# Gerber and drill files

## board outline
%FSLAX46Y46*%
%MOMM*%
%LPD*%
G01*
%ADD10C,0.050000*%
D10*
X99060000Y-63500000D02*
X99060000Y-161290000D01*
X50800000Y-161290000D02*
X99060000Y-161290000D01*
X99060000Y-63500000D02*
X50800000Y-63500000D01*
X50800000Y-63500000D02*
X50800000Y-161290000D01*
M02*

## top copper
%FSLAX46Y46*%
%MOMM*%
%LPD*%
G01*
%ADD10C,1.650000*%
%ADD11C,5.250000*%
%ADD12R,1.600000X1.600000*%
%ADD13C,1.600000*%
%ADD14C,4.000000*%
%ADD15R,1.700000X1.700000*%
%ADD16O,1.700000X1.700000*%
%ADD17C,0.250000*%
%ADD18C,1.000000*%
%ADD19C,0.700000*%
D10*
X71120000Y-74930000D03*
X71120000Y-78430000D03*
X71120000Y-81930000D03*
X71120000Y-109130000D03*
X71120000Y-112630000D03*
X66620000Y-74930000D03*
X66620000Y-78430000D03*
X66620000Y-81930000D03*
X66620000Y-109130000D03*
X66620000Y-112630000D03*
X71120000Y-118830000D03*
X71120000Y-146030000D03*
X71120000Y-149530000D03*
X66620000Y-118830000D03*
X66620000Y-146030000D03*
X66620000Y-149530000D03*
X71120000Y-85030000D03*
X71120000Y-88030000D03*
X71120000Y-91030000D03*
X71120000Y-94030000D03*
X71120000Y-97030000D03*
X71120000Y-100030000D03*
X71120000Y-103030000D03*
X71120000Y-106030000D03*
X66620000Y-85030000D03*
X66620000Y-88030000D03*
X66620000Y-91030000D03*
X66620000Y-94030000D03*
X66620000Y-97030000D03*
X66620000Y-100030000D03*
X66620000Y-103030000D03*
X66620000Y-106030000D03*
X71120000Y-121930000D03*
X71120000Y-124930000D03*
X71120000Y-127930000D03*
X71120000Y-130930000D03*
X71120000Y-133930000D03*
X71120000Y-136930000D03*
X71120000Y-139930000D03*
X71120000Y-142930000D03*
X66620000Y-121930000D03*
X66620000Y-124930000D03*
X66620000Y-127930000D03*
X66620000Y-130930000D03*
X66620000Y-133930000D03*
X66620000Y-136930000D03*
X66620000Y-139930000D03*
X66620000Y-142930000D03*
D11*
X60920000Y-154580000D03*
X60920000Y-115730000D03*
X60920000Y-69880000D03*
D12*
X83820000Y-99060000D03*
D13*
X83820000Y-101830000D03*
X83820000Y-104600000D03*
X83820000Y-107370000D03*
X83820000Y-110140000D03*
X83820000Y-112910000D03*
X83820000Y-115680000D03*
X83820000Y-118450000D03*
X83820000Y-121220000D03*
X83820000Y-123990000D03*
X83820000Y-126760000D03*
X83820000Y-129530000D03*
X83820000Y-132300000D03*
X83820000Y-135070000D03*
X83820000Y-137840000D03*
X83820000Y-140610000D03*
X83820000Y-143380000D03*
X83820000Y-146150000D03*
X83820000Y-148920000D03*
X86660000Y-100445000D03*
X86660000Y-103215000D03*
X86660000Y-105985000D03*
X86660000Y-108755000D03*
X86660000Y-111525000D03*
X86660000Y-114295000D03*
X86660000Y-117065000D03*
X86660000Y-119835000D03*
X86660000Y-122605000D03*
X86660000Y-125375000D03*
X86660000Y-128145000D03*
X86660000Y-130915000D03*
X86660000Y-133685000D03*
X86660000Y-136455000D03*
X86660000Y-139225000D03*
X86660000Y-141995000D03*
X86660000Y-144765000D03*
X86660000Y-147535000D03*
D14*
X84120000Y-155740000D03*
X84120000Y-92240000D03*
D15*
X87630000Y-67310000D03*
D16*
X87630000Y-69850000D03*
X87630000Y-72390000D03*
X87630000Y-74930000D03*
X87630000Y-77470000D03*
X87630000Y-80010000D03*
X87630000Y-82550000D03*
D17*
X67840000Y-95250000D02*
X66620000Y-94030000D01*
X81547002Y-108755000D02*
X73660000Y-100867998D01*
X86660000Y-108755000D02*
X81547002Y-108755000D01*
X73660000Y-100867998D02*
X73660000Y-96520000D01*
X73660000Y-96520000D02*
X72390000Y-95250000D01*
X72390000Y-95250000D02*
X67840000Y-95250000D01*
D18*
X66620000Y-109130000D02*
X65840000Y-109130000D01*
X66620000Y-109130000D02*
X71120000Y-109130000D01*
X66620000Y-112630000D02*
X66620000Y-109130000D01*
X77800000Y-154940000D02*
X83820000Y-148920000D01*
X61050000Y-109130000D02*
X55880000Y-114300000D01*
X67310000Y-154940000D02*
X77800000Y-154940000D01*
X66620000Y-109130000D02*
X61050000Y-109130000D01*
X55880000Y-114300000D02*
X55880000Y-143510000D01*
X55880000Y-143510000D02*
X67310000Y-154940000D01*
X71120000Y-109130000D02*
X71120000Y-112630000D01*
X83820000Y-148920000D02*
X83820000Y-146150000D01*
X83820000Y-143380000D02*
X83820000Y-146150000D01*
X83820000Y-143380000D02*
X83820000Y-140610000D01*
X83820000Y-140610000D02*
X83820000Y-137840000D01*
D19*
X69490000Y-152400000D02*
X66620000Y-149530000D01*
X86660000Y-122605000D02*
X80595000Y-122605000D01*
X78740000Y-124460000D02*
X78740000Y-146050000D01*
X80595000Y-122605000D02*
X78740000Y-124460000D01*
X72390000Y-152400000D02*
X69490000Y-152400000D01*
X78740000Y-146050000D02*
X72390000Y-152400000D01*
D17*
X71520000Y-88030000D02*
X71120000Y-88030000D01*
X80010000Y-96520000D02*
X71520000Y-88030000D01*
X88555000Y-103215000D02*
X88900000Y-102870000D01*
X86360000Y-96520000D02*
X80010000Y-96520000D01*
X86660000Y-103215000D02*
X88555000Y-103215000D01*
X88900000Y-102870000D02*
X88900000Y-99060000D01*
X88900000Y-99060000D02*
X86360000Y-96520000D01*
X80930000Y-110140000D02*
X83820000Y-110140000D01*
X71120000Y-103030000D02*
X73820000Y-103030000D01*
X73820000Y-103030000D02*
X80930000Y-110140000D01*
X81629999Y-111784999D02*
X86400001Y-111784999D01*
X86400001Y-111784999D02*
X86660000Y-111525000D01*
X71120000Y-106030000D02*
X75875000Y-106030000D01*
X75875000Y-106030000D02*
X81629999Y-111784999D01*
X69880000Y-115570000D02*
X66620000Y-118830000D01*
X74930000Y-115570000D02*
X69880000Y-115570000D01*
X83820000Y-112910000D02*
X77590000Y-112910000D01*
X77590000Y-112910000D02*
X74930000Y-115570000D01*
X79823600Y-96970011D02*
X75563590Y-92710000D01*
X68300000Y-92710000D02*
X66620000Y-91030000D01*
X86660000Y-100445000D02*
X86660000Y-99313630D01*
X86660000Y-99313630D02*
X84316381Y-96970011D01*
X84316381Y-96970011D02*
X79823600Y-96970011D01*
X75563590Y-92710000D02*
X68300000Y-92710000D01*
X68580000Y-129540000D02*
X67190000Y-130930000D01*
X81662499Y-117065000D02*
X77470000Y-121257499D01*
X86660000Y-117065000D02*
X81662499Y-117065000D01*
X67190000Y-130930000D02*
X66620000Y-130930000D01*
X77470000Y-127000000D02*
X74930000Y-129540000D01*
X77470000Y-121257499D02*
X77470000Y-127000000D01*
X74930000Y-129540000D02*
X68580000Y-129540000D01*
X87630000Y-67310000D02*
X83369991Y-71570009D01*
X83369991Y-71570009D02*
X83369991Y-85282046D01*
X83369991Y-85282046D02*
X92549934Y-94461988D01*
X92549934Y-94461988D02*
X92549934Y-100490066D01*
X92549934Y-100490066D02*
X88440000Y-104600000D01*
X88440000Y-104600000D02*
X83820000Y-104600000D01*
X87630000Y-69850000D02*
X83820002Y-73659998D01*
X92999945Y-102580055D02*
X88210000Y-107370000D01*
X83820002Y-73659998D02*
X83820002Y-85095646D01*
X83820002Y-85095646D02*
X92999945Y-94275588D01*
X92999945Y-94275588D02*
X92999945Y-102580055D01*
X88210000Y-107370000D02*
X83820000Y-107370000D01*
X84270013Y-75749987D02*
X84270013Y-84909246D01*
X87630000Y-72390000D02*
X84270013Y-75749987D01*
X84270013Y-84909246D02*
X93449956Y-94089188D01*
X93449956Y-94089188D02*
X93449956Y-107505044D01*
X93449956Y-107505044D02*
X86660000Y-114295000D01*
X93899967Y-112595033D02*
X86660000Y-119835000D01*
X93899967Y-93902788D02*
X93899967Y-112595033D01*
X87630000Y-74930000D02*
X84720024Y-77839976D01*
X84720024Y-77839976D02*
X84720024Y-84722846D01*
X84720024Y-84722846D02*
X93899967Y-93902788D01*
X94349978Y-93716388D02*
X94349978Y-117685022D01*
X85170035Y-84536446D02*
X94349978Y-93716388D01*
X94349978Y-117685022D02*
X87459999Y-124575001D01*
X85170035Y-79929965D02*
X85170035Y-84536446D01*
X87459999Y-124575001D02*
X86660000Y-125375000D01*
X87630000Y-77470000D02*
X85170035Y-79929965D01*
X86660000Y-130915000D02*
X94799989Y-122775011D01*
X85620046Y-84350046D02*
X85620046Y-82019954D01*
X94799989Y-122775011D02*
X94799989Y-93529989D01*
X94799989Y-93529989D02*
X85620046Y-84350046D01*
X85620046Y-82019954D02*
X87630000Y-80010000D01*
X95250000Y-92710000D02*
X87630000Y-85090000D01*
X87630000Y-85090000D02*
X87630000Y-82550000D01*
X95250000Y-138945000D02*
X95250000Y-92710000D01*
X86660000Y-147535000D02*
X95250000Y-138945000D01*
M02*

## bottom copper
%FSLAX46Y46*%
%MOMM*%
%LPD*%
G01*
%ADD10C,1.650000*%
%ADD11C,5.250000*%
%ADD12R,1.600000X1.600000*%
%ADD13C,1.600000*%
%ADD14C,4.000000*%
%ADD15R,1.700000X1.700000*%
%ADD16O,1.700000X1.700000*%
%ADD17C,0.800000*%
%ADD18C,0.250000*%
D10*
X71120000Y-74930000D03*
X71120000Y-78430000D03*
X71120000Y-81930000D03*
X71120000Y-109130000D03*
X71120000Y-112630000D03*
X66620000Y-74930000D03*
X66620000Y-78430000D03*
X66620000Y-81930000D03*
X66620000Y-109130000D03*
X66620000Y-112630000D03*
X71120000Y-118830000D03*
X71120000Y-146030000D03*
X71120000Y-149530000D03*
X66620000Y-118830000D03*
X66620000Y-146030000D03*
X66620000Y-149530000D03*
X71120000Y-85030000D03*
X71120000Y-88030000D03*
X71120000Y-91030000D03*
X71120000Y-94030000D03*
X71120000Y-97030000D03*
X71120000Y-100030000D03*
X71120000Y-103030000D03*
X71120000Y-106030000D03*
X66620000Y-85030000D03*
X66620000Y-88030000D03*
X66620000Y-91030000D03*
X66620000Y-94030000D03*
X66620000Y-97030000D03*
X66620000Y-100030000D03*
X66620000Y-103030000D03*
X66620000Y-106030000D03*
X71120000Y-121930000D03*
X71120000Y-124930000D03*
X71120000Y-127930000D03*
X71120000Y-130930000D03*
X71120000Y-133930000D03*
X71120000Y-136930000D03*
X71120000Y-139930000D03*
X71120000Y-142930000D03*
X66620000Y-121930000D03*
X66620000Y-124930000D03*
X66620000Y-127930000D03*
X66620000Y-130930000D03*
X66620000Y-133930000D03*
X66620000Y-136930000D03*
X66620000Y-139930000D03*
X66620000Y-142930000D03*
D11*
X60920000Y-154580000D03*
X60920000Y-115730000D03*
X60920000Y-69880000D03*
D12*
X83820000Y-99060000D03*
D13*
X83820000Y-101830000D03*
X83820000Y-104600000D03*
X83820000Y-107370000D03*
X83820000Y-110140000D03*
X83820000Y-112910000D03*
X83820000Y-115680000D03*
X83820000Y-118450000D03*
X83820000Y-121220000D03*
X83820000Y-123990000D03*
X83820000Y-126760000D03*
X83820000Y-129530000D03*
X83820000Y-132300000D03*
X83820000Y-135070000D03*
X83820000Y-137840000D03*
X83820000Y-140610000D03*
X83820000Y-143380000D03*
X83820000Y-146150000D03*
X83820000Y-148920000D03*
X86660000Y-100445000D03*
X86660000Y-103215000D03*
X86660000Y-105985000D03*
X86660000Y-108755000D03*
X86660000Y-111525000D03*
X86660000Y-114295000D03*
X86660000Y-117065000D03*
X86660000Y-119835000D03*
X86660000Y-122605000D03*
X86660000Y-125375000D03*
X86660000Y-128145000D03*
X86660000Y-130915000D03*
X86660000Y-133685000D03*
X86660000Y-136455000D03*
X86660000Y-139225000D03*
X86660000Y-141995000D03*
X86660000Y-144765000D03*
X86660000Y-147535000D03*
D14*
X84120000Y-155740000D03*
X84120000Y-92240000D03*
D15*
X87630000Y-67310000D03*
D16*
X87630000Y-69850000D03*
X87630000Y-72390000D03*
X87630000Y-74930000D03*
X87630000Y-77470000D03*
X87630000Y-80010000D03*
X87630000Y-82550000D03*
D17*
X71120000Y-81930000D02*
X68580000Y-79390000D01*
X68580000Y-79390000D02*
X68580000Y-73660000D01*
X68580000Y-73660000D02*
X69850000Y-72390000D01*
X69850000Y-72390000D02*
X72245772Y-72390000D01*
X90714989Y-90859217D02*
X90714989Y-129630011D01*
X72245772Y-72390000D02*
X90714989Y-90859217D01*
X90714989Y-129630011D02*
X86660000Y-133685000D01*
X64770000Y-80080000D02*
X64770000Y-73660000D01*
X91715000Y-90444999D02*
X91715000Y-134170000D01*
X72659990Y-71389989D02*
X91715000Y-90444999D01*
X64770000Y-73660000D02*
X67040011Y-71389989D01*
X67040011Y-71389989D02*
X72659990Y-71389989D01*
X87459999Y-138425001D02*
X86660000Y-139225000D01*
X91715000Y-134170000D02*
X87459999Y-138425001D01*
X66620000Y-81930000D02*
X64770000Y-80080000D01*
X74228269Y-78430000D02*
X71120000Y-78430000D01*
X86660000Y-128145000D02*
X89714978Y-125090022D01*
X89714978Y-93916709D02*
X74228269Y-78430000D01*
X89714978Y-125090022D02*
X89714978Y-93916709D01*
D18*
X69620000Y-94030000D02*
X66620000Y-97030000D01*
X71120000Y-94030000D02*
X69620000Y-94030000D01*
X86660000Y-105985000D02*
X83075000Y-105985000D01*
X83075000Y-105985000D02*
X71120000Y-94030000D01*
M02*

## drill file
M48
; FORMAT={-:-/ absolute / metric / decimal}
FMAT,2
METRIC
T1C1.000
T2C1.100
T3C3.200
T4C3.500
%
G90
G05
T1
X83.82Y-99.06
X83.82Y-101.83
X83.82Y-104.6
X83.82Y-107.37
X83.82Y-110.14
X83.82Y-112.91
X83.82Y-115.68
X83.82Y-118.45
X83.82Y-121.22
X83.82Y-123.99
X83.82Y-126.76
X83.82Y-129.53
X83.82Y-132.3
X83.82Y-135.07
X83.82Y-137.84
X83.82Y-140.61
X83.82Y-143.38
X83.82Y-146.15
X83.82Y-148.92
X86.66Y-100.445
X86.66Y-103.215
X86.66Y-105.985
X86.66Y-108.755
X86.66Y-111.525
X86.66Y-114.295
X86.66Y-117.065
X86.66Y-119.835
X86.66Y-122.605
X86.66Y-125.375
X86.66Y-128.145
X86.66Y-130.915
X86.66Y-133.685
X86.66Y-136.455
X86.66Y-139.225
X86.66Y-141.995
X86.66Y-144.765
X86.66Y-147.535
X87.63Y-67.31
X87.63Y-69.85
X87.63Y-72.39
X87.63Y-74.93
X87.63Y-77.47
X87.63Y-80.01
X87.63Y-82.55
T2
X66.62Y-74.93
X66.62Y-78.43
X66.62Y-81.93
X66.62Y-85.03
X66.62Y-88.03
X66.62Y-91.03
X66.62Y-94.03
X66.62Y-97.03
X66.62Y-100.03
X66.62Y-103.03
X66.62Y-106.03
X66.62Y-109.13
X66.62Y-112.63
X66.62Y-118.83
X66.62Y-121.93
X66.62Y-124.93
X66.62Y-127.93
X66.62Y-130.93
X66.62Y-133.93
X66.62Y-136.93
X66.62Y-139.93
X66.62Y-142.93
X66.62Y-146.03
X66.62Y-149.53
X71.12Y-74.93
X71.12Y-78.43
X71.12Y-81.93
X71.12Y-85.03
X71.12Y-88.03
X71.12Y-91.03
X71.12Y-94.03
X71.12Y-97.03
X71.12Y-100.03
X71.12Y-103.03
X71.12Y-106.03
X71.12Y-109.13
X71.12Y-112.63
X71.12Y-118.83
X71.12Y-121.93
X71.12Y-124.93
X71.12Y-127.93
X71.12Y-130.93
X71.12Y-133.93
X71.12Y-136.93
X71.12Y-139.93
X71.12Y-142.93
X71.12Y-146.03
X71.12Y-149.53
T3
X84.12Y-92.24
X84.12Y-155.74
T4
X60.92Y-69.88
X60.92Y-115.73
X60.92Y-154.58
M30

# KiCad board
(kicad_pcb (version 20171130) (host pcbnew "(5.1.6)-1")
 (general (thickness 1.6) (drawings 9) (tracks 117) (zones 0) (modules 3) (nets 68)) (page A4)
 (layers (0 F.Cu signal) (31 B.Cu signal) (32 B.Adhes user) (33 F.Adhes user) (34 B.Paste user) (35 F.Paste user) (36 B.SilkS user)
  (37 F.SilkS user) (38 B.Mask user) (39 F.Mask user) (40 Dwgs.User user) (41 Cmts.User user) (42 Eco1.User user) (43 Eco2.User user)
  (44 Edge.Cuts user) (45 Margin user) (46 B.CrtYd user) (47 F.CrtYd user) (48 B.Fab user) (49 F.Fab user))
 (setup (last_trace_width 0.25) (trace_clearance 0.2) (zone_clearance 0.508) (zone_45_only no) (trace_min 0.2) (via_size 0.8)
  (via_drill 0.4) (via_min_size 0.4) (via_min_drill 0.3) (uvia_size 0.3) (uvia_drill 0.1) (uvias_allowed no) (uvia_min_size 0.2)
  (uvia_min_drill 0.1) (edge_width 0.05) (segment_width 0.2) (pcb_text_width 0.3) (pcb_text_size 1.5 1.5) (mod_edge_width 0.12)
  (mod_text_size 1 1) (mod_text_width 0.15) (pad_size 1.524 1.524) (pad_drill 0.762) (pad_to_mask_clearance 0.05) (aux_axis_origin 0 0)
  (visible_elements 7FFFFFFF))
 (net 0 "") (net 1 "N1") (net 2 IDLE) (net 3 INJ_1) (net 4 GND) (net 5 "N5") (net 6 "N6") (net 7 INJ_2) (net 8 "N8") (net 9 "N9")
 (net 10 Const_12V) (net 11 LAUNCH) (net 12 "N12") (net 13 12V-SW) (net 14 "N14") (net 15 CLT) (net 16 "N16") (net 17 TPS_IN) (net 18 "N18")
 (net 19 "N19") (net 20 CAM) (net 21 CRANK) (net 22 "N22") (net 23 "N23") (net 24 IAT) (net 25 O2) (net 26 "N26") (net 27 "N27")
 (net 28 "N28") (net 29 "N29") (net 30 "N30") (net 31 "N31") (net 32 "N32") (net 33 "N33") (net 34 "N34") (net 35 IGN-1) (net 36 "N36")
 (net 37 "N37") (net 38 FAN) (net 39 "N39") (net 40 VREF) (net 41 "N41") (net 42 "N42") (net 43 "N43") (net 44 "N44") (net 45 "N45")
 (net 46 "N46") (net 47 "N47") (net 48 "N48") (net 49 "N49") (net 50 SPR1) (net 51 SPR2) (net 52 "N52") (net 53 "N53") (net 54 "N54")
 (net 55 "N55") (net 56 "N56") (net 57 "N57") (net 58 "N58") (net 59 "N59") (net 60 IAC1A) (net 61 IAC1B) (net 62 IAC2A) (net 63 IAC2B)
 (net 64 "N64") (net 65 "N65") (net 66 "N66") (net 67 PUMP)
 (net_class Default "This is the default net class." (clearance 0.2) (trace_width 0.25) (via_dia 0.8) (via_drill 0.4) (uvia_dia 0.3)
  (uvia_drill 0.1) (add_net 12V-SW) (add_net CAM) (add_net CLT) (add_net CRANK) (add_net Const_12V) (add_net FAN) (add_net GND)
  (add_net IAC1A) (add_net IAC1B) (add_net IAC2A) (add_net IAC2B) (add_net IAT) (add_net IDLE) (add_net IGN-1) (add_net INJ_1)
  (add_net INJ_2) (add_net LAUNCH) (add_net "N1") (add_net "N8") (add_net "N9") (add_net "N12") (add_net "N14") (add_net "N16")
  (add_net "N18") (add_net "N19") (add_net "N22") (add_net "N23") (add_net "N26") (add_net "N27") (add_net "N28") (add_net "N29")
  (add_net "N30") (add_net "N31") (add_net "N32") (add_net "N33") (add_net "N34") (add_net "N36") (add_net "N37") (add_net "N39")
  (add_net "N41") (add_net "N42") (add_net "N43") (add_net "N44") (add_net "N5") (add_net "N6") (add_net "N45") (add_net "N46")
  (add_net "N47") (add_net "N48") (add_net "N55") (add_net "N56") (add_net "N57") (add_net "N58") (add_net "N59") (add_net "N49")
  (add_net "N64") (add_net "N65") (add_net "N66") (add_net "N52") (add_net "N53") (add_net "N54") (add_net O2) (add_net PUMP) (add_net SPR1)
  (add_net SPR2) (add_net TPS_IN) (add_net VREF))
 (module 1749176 (layer F.Cu) (at 71.12 74.93 180)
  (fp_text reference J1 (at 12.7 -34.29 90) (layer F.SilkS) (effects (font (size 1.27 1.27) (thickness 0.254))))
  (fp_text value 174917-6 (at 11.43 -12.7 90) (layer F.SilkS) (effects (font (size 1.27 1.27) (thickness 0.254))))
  (pad 1 thru_hole circle (at 0 0 270) (size 1.65 1.65) (drill 1.1) (layers *.Cu *.Mask F.SilkS) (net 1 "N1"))
  (pad 2 thru_hole circle (at 0 -3.5 270) (size 1.65 1.65) (drill 1.1) (layers *.Cu *.Mask F.SilkS) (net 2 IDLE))
  (pad 3 thru_hole circle (at 0 -7 270) (size 1.65 1.65) (drill 1.1) (layers *.Cu *.Mask F.SilkS) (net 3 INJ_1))
  (pad 4 thru_hole circle (at 0 -34.2 270) (size 1.65 1.65) (drill 1.1) (layers *.Cu *.Mask F.SilkS) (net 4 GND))
  (pad 5 thru_hole circle (at 0 -37.7 270) (size 1.65 1.65) (drill 1.1) (layers *.Cu *.Mask F.SilkS) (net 4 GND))
  (pad 6 thru_hole circle (at 4.5 0 270) (size 1.65 1.65) (drill 1.1) (layers *.Cu *.Mask F.SilkS) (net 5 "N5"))
  (pad 7 thru_hole circle (at 4.5 -3.5 270) (size 1.65 1.65) (drill 1.1) (layers *.Cu *.Mask F.SilkS) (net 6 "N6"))
  (pad 8 thru_hole circle (at 4.5 -7 270) (size 1.65 1.65) (drill 1.1) (layers *.Cu *.Mask F.SilkS) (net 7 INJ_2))
  (pad 9 thru_hole circle (at 4.5 -34.2 270) (size 1.65 1.65) (drill 1.1) (layers *.Cu *.Mask F.SilkS) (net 4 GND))
  (pad 10 thru_hole circle (at 4.5 -37.7 270) (size 1.65 1.65) (drill 1.1) (layers *.Cu *.Mask F.SilkS) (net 4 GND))
  (pad 11 thru_hole circle (at 0 -43.9 270) (size 1.65 1.65) (drill 1.1) (layers *.Cu *.Mask F.SilkS) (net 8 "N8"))
  (pad 12 thru_hole circle (at 0 -71.1 270) (size 1.65 1.65) (drill 1.1) (layers *.Cu *.Mask F.SilkS) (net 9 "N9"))
  (pad 13 thru_hole circle (at 0 -74.6 270) (size 1.65 1.65) (drill 1.1) (layers *.Cu *.Mask F.SilkS) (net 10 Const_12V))
  (pad 14 thru_hole circle (at 4.5 -43.9 270) (size 1.65 1.65) (drill 1.1) (layers *.Cu *.Mask F.SilkS) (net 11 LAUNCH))
  (pad 15 thru_hole circle (at 4.5 -71.1 270) (size 1.65 1.65) (drill 1.1) (layers *.Cu *.Mask F.SilkS) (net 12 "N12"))
  (pad 16 thru_hole circle (at 4.5 -74.6 270) (size 1.65 1.65) (drill 1.1) (layers *.Cu *.Mask F.SilkS) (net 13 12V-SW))
  (pad 17 thru_hole circle (at 0 -10.1 270) (size 1.65 1.65) (drill 1.1) (layers *.Cu *.Mask F.SilkS) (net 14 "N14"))
  (pad 18 thru_hole circle (at 0 -13.1 270) (size 1.65 1.65) (drill 1.1) (layers *.Cu *.Mask F.SilkS) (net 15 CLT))
  (pad 19 thru_hole circle (at 0 -16.1 270) (size 1.65 1.65) (drill 1.1) (layers *.Cu *.Mask F.SilkS) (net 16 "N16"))
  (pad 20 thru_hole circle (at 0 -19.1 270) (size 1.65 1.65) (drill 1.1) (layers *.Cu *.Mask F.SilkS) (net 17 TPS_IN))
  (pad 21 thru_hole circle (at 0 -22.1 270) (size 1.65 1.65) (drill 1.1) (layers *.Cu *.Mask F.SilkS) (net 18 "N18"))
  (pad 22 thru_hole circle (at 0 -25.1 270) (size 1.65 1.65) (drill 1.1) (layers *.Cu *.Mask F.SilkS) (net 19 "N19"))
  (pad 23 thru_hole circle (at 0 -28.1 270) (size 1.65 1.65) (drill 1.1) (layers *.Cu *.Mask F.SilkS) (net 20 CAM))
  (pad 24 thru_hole circle (at 0 -31.1 270) (size 1.65 1.65) (drill 1.1) (layers *.Cu *.Mask F.SilkS) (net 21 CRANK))
  (pad 25 thru_hole circle (at 4.5 -10.1 270) (size 1.65 1.65) (drill 1.1) (layers *.Cu *.Mask F.SilkS) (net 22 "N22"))
  (pad 26 thru_hole circle (at 4.5 -13.1 270) (size 1.65 1.65) (drill 1.1) (layers *.Cu *.Mask F.SilkS) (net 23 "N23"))
  (pad 27 thru_hole circle (at 4.5 -16.1 270) (size 1.65 1.65) (drill 1.1) (layers *.Cu *.Mask F.SilkS) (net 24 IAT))
  (pad 28 thru_hole circle (at 4.5 -19.1 270) (size 1.65 1.65) (drill 1.1) (layers *.Cu *.Mask F.SilkS) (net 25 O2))
  (pad 29 thru_hole circle (at 4.5 -22.1 270) (size 1.65 1.65) (drill 1.1) (layers *.Cu *.Mask F.SilkS) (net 17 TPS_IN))
  (pad 30 thru_hole circle (at 4.5 -25.1 270) (size 1.65 1.65) (drill 1.1) (layers *.Cu *.Mask F.SilkS) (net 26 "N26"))
  (pad 31 thru_hole circle (at 4.5 -28.1 270) (size 1.65 1.65) (drill 1.1) (layers *.Cu *.Mask F.SilkS) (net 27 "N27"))
  (pad 32 thru_hole circle (at 4.5 -31.1 270) (size 1.65 1.65) (drill 1.1) (layers *.Cu *.Mask F.SilkS) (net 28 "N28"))
  (pad 33 thru_hole circle (at 0 -47 270) (size 1.65 1.65) (drill 1.1) (layers *.Cu *.Mask F.SilkS) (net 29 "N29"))
  (pad 34 thru_hole circle (at 0 -50 270) (size 1.65 1.65) (drill 1.1) (layers *.Cu *.Mask F.SilkS) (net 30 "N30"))
  (pad 35 thru_hole circle (at 0 -53 270) (size 1.65 1.65) (drill 1.1) (layers *.Cu *.Mask F.SilkS) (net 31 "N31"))
  (pad 36 thru_hole circle (at 0 -56 270) (size 1.65 1.65) (drill 1.1) (layers *.Cu *.Mask F.SilkS) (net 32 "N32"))
  (pad 37 thru_hole circle (at 0 -59 270) (size 1.65 1.65) (drill 1.1) (layers *.Cu *.Mask F.SilkS) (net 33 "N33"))
  (pad 38 thru_hole circle (at 0 -62 270) (size 1.65 1.65) (drill 1.1) (layers *.Cu *.Mask F.SilkS) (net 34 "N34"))
  (pad 39 thru_hole circle (at 0 -65 270) (size 1.65 1.65) (drill 1.1) (layers *.Cu *.Mask F.SilkS) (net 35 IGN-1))
  (pad 40 thru_hole circle (at 0 -68 270) (size 1.65 1.65) (drill 1.1) (layers *.Cu *.Mask F.SilkS) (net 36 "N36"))
  (pad 41 thru_hole circle (at 4.5 -47 270) (size 1.65 1.65) (drill 1.1) (layers *.Cu *.Mask F.SilkS) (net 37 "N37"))
  (pad 42 thru_hole circle (at 4.5 -50 270) (size 1.65 1.65) (drill 1.1) (layers *.Cu *.Mask F.SilkS) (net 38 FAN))
  (pad 43 thru_hole circle (at 4.5 -53 270) (size 1.65 1.65) (drill 1.1) (layers *.Cu *.Mask F.SilkS) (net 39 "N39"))
  (pad 44 thru_hole circle (at 4.5 -56 270) (size 1.65 1.65) (drill 1.1) (layers *.Cu *.Mask F.SilkS) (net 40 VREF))
  (pad 45 thru_hole circle (at 4.5 -59 270) (size 1.65 1.65) (drill 1.1) (layers *.Cu *.Mask F.SilkS) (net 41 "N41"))
  (pad 46 thru_hole circle (at 4.5 -62 270) (size 1.65 1.65) (drill 1.1) (layers *.Cu *.Mask F.SilkS) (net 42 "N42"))
  (pad 47 thru_hole circle (at 4.5 -65 270) (size 1.65 1.65) (drill 1.1) (layers *.Cu *.Mask F.SilkS) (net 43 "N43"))
  (pad 48 thru_hole circle (at 4.5 -68 270) (size 1.65 1.65) (drill 1.1) (layers *.Cu *.Mask F.SilkS) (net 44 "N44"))
  (pad MH1 thru_hole circle (at 10.2 -79.65 270) (size 5.25 5.25) (drill 3.5) (layers *.Cu *.Mask F.SilkS) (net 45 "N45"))
  (pad MH2 thru_hole circle (at 10.2 -40.8 270) (size 5.25 5.25) (drill 3.5) (layers *.Cu *.Mask F.SilkS) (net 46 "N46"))
  (pad MH3 thru_hole circle (at 10.2 5.05 270) (size 5.25 5.25) (drill 3.5) (layers *.Cu *.Mask F.SilkS) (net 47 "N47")))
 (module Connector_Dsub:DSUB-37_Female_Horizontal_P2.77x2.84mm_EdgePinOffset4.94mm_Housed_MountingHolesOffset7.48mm (layer F.Cu)
  (at 83.82 99.06 90)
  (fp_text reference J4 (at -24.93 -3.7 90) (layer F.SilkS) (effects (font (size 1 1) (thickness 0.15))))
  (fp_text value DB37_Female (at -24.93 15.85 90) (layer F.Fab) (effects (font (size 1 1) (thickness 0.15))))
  (pad 1 thru_hole rect (at 0 0 90) (size 1.6 1.6) (drill 1) (layers *.Cu *.Mask) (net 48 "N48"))
  (pad 2 thru_hole circle (at -2.77 0 90) (size 1.6 1.6) (drill 1) (layers *.Cu *.Mask) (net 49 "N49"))
  (pad 3 thru_hole circle (at -5.54 0 90) (size 1.6 1.6) (drill 1) (layers *.Cu *.Mask) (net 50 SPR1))
  (pad 4 thru_hole circle (at -8.31 0 90) (size 1.6 1.6) (drill 1) (layers *.Cu *.Mask) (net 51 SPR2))
  (pad 5 thru_hole circle (at -11.08 0 90) (size 1.6 1.6) (drill 1) (layers *.Cu *.Mask) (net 20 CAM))
  (pad 6 thru_hole circle (at -13.85 0 90) (size 1.6 1.6) (drill 1) (layers *.Cu *.Mask) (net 11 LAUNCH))
  (pad 7 thru_hole circle (at -16.62 0 90) (size 1.6 1.6) (drill 1) (layers *.Cu *.Mask) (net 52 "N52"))
  (pad 8 thru_hole circle (at -19.39 0 90) (size 1.6 1.6) (drill 1) (layers *.Cu *.Mask) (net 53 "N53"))
  (pad 9 thru_hole circle (at -22.16 0 90) (size 1.6 1.6) (drill 1) (layers *.Cu *.Mask) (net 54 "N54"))
  (pad 10 thru_hole circle (at -24.93 0 90) (size 1.6 1.6) (drill 1) (layers *.Cu *.Mask) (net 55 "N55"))
  (pad 11 thru_hole circle (at -27.7 0 90) (size 1.6 1.6) (drill 1) (layers *.Cu *.Mask) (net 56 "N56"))
  (pad 12 thru_hole circle (at -30.47 0 90) (size 1.6 1.6) (drill 1) (layers *.Cu *.Mask) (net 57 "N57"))
  (pad 13 thru_hole circle (at -33.24 0 90) (size 1.6 1.6) (drill 1) (layers *.Cu *.Mask) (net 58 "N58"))
  (pad 14 thru_hole circle (at -36.01 0 90) (size 1.6 1.6) (drill 1) (layers *.Cu *.Mask) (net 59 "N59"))
  (pad 15 thru_hole circle (at -38.78 0 90) (size 1.6 1.6) (drill 1) (layers *.Cu *.Mask) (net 4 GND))
  (pad 16 thru_hole circle (at -41.55 0 90) (size 1.6 1.6) (drill 1) (layers *.Cu *.Mask) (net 4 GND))
  (pad 17 thru_hole circle (at -44.32 0 90) (size 1.6 1.6) (drill 1) (layers *.Cu *.Mask) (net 4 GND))
  (pad 18 thru_hole circle (at -47.09 0 90) (size 1.6 1.6) (drill 1) (layers *.Cu *.Mask) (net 4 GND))
  (pad 19 thru_hole circle (at -49.86 0 90) (size 1.6 1.6) (drill 1) (layers *.Cu *.Mask) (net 4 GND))
  (pad 20 thru_hole circle (at -1.385 2.84 90) (size 1.6 1.6) (drill 1) (layers *.Cu *.Mask) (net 24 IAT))
  (pad 21 thru_hole circle (at -4.155 2.84 90) (size 1.6 1.6) (drill 1) (layers *.Cu *.Mask) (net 15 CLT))
  (pad 22 thru_hole circle (at -6.925 2.84 90) (size 1.6 1.6) (drill 1) (layers *.Cu *.Mask) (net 17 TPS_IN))
  (pad 23 thru_hole circle (at -9.695 2.84 90) (size 1.6 1.6) (drill 1) (layers *.Cu *.Mask) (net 25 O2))
  (pad 24 thru_hole circle (at -12.465 2.84 90) (size 1.6 1.6) (drill 1) (layers *.Cu *.Mask) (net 21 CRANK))
  (pad 25 thru_hole circle (at -15.235 2.84 90) (size 1.6 1.6) (drill 1) (layers *.Cu *.Mask) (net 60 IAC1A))
  (pad 26 thru_hole circle (at -18.005 2.84 90) (size 1.6 1.6) (drill 1) (layers *.Cu *.Mask) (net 40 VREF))
  (pad 27 thru_hole circle (at -20.775 2.84 90) (size 1.6 1.6) (drill 1) (layers *.Cu *.Mask) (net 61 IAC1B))
  (pad 28 thru_hole circle (at -23.545 2.84 90) (size 1.6 1.6) (drill 1) (layers *.Cu *.Mask) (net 13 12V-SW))
  (pad 29 thru_hole circle (at -26.315 2.84 90) (size 1.6 1.6) (drill 1) (layers *.Cu *.Mask) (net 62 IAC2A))
  (pad 30 thru_hole circle (at -29.085 2.84 90) (size 1.6 1.6) (drill 1) (layers *.Cu *.Mask) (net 2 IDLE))
  (pad 31 thru_hole circle (at -31.855 2.84 90) (size 1.6 1.6) (drill 1) (layers *.Cu *.Mask) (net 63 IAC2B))
  (pad 32 thru_hole circle (at -34.625 2.84 90) (size 1.6 1.6) (drill 1) (layers *.Cu *.Mask) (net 3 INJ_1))
  (pad 33 thru_hole circle (at -37.395 2.84 90) (size 1.6 1.6) (drill 1) (layers *.Cu *.Mask) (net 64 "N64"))
  (pad 34 thru_hole circle (at -40.165 2.84 90) (size 1.6 1.6) (drill 1) (layers *.Cu *.Mask) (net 7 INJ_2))
  (pad 35 thru_hole circle (at -42.935 2.84 90) (size 1.6 1.6) (drill 1) (layers *.Cu *.Mask) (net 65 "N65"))
  (pad 36 thru_hole circle (at -45.705 2.84 90) (size 1.6 1.6) (drill 1) (layers *.Cu *.Mask) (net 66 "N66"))
  (pad 37 thru_hole circle (at -48.475 2.84 90) (size 1.6 1.6) (drill 1) (layers *.Cu *.Mask) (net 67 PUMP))
  (pad 0 thru_hole circle (at -56.68 0.3 90) (size 4 4) (drill 3.2) (layers *.Cu *.Mask))
  (pad 0 thru_hole circle (at 6.82 0.3 90) (size 4 4) (drill 3.2) (layers *.Cu *.Mask)))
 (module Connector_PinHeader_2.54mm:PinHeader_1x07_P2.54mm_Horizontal (layer F.Cu) (at 87.63 67.31)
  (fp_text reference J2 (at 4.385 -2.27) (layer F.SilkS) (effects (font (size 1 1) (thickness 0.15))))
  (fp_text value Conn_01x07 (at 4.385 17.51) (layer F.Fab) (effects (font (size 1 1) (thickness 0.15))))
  (pad 1 thru_hole rect (at 0 0) (size 1.7 1.7) (drill 1) (layers *.Cu *.Mask) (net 50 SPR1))
  (pad 2 thru_hole oval (at 0 2.54) (size 1.7 1.7) (drill 1) (layers *.Cu *.Mask) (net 51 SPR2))
  (pad 3 thru_hole oval (at 0 5.08) (size 1.7 1.7) (drill 1) (layers *.Cu *.Mask) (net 60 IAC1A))
  (pad 4 thru_hole oval (at 0 7.62) (size 1.7 1.7) (drill 1) (layers *.Cu *.Mask) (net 61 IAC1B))
  (pad 5 thru_hole oval (at 0 10.16) (size 1.7 1.7) (drill 1) (layers *.Cu *.Mask) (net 62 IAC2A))
  (pad 6 thru_hole oval (at 0 12.7) (size 1.7 1.7) (drill 1) (layers *.Cu *.Mask) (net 63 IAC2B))
  (pad 7 thru_hole oval (at 0 15.24) (size 1.7 1.7) (drill 1) (layers *.Cu *.Mask) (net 67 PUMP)))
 (gr_line (start 99.06 63.5) (end 99.06 161.29) (layer Edge.Cuts) (width 0.05))
 (gr_line (start 50.8 161.29) (end 99.06 161.29) (layer Edge.Cuts) (width 0.05))
 (gr_line (start 99.06 63.5) (end 50.8 63.5) (layer Edge.Cuts) (width 0.05))
 (gr_line (start 50.8 63.5) (end 50.8 161.29) (layer Edge.Cuts) (width 0.05))
 (segment (start 71.12 81.93) (end 68.58 79.39) (width 0.8) (layer B.Cu) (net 3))
 (segment (start 68.58 79.39) (end 68.58 73.66) (width 0.8) (layer B.Cu) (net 3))
 (segment (start 68.58 73.66) (end 69.85 72.39) (width 0.8) (layer B.Cu) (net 3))
 (segment (start 69.85 72.39) (end 72.245772 72.39) (width 0.8) (layer B.Cu) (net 3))
 (segment (start 90.714989 90.859217) (end 90.714989 129.630011) (width 0.8) (layer B.Cu) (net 3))
 (segment (start 72.245772 72.39) (end 90.714989 90.859217) (width 0.8) (layer B.Cu) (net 3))
 (segment (start 90.714989 129.630011) (end 86.66 133.685) (width 0.8) (layer B.Cu) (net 3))
 (segment (start 64.77 80.08) (end 64.77 73.66) (width 0.8) (layer B.Cu) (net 7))
 (segment (start 91.715 90.444999) (end 91.715 134.17) (width 0.8) (layer B.Cu) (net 7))
 (segment (start 72.65999 71.389989) (end 91.715 90.444999) (width 0.8) (layer B.Cu) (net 7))
 (segment (start 64.77 73.66) (end 67.040011 71.389989) (width 0.8) (layer B.Cu) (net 7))
 (segment (start 67.040011 71.389989) (end 72.65999 71.389989) (width 0.8) (layer B.Cu) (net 7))
 (segment (start 87.459999 138.425001) (end 86.66 139.225) (width 0.8) (layer B.Cu) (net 7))
 (segment (start 91.715 134.17) (end 87.459999 138.425001) (width 0.8) (layer B.Cu) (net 7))
 (segment (start 66.62 81.93) (end 64.77 80.08) (width 0.8) (layer B.Cu) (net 7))
 (segment (start 67.84 95.25) (end 66.62 94.03) (width 0.25) (layer F.Cu) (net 25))
 (segment (start 81.547002 108.755) (end 73.66 100.867998) (width 0.25) (layer F.Cu) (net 25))
 (segment (start 86.66 108.755) (end 81.547002 108.755) (width 0.25) (layer F.Cu) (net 25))
 (segment (start 73.66 100.867998) (end 73.66 96.52) (width 0.25) (layer F.Cu) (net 25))
 (segment (start 73.66 96.52) (end 72.39 95.25) (width 0.25) (layer F.Cu) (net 25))
 (segment (start 72.39 95.25) (end 67.84 95.25) (width 0.25) (layer F.Cu) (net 25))
 (segment (start 66.62 109.13) (end 65.84 109.13) (width 1) (layer F.Cu) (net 4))
 (segment (start 66.62 109.13) (end 71.12 109.13) (width 1) (layer F.Cu) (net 4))
 (segment (start 66.62 112.63) (end 66.62 109.13) (width 1) (layer F.Cu) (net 4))
 (segment (start 77.8 154.94) (end 83.82 148.92) (width 1) (layer F.Cu) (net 4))
 (segment (start 61.05 109.13) (end 55.88 114.3) (width 1) (layer F.Cu) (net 4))
 (segment (start 67.31 154.94) (end 77.8 154.94) (width 1) (layer F.Cu) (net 4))
 (segment (start 66.62 109.13) (end 61.05 109.13) (width 1) (layer F.Cu) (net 4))
 (segment (start 55.88 114.3) (end 55.88 143.51) (width 1) (layer F.Cu) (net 4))
 (segment (start 55.88 143.51) (end 67.31 154.94) (width 1) (layer F.Cu) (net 4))
 (segment (start 71.12 109.13) (end 71.12 112.63) (width 1) (layer F.Cu) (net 4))
 (segment (start 83.82 148.92) (end 83.82 146.15) (width 1) (layer F.Cu) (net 4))
 (segment (start 83.82 143.38) (end 83.82 146.15) (width 1) (layer F.Cu) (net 4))
 (segment (start 83.82 143.38) (end 83.82 140.61) (width 1) (layer F.Cu) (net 4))
 (segment (start 83.82 140.61) (end 83.82 137.84) (width 1) (layer F.Cu) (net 4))
 (segment (start 69.49 152.4) (end 66.62 149.53) (width 0.7) (layer F.Cu) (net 13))
 (segment (start 86.66 122.605) (end 80.595 122.605) (width 0.7) (layer F.Cu) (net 13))
 (segment (start 78.74 124.46) (end 78.74 146.05) (width 0.7) (layer F.Cu) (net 13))
 (segment (start 80.595 122.605) (end 78.74 124.46) (width 0.7) (layer F.Cu) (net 13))
 (segment (start 72.39 152.4) (end 69.49 152.4) (width 0.7) (layer F.Cu) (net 13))
 (segment (start 78.74 146.05) (end 72.39 152.4) (width 0.7) (layer F.Cu) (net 13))
 (segment (start 71.52 88.03) (end 71.12 88.03) (width 0.25) (layer F.Cu) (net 15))
 (segment (start 80.01 96.52) (end 71.52 88.03) (width 0.25) (layer F.Cu) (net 15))
 (segment (start 88.555 103.215) (end 88.9 102.87) (width 0.25) (layer F.Cu) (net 15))
 (segment (start 86.36 96.52) (end 80.01 96.52) (width 0.25) (layer F.Cu) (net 15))
 (segment (start 86.66 103.215) (end 88.555 103.215) (width 0.25) (layer F.Cu) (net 15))
 (segment (start 88.9 102.87) (end 88.9 99.06) (width 0.25) (layer F.Cu) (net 15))
 (segment (start 88.9 99.06) (end 86.36 96.52) (width 0.25) (layer F.Cu) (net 15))
 (segment (start 80.93 110.14) (end 83.82 110.14) (width 0.25) (layer F.Cu) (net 20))
 (segment (start 71.12 103.03) (end 73.82 103.03) (width 0.25) (layer F.Cu) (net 20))
 (segment (start 73.82 103.03) (end 80.93 110.14) (width 0.25) (layer F.Cu) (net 20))
 (segment (start 81.629999 111.784999) (end 86.400001 111.784999) (width 0.25) (layer F.Cu) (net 21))
 (segment (start 86.400001 111.784999) (end 86.66 111.525) (width 0.25) (layer F.Cu) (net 21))
 (segment (start 71.12 106.03) (end 75.875 106.03) (width 0.25) (layer F.Cu) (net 21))
 (segment (start 75.875 106.03) (end 81.629999 111.784999) (width 0.25) (layer F.Cu) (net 21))
 (segment (start 74.228269 78.43) (end 71.12 78.43) (width 0.8) (layer B.Cu) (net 2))
 (segment (start 86.66 128.145) (end 89.714978 125.090022) (width 0.8) (layer B.Cu) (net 2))
 (segment (start 89.714978 93.916709) (end 74.228269 78.43) (width 0.8) (layer B.Cu) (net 2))
 (segment (start 89.714978 125.090022) (end 89.714978 93.916709) (width 0.8) (layer B.Cu) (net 2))
 (segment (start 69.88 115.57) (end 66.62 118.83) (width 0.25) (layer F.Cu) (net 11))
 (segment (start 74.93 115.57) (end 69.88 115.57) (width 0.25) (layer F.Cu) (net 11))
 (segment (start 83.82 112.91) (end 77.59 112.91) (width 0.25) (layer F.Cu) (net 11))
 (segment (start 77.59 112.91) (end 74.93 115.57) (width 0.25) (layer F.Cu) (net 11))
 (segment (start 69.62 94.03) (end 66.62 97.03) (width 0.25) (layer B.Cu) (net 17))
 (segment (start 71.12 94.03) (end 69.62 94.03) (width 0.25) (layer B.Cu) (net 17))
 (segment (start 86.66 105.985) (end 83.075 105.985) (width 0.25) (layer B.Cu) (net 17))
 (segment (start 83.075 105.985) (end 71.12 94.03) (width 0.25) (layer B.Cu) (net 17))
 (segment (start 79.8236 96.970011) (end 75.56359 92.71) (width 0.25) (layer F.Cu) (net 24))
 (segment (start 68.3 92.71) (end 66.62 91.03) (width 0.25) (layer F.Cu) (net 24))
 (segment (start 86.66 100.445) (end 86.66 99.31363) (width 0.25) (layer F.Cu) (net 24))
 (segment (start 86.66 99.31363) (end 84.316381 96.970011) (width 0.25) (layer F.Cu) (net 24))
 (segment (start 84.316381 96.970011) (end 79.8236 96.970011) (width 0.25) (layer F.Cu) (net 24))
 (segment (start 75.56359 92.71) (end 68.3 92.71) (width 0.25) (layer F.Cu) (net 24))
 (segment (start 68.58 129.54) (end 67.19 130.93) (width 0.25) (layer F.Cu) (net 40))
 (segment (start 81.662499 117.065) (end 77.47 121.257499) (width 0.25) (layer F.Cu) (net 40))
 (segment (start 86.66 117.065) (end 81.662499 117.065) (width 0.25) (layer F.Cu) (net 40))
 (segment (start 67.19 130.93) (end 66.62 130.93) (width 0.25) (layer F.Cu) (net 40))
 (segment (start 77.47 127) (end 74.93 129.54) (width 0.25) (layer F.Cu) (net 40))
 (segment (start 77.47 121.257499) (end 77.47 127) (width 0.25) (layer F.Cu) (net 40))
 (segment (start 74.93 129.54) (end 68.58 129.54) (width 0.25) (layer F.Cu) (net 40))
 (segment (start 87.63 67.31) (end 83.369991 71.570009) (width 0.25) (layer F.Cu) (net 50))
 (segment (start 83.369991 71.570009) (end 83.369991 85.282046) (width 0.25) (layer F.Cu) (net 50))
 (segment (start 83.369991 85.282046) (end 92.549934 94.461988) (width 0.25) (layer F.Cu) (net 50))
 (segment (start 92.549934 94.461988) (end 92.549934 100.490066) (width 0.25) (layer F.Cu) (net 50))
 (segment (start 92.549934 100.490066) (end 88.44 104.6) (width 0.25) (layer F.Cu) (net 50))
 (segment (start 88.44 104.6) (end 83.82 104.6) (width 0.25) (layer F.Cu) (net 50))
 (segment (start 87.63 69.85) (end 83.820002 73.659998) (width 0.25) (layer F.Cu) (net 51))
 (segment (start 92.999945 102.580055) (end 88.21 107.37) (width 0.25) (layer F.Cu) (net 51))
 (segment (start 83.820002 73.659998) (end 83.820002 85.095646) (width 0.25) (layer F.Cu) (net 51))
 (segment (start 83.820002 85.095646) (end 92.999945 94.275588) (width 0.25) (layer F.Cu) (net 51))
 (segment (start 92.999945 94.275588) (end 92.999945 102.580055) (width 0.25) (layer F.Cu) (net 51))
 (segment (start 88.21 107.37) (end 83.82 107.37) (width 0.25) (layer F.Cu) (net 51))
 (segment (start 84.270013 75.749987) (end 84.270013 84.909246) (width 0.25) (layer F.Cu) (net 60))
 (segment (start 87.63 72.39) (end 84.270013 75.749987) (width 0.25) (layer F.Cu) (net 60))
 (segment (start 84.270013 84.909246) (end 93.449956 94.089188) (width 0.25) (layer F.Cu) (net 60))
 (segment (start 93.449956 94.089188) (end 93.449956 107.505044) (width 0.25) (layer F.Cu) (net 60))
 (segment (start 93.449956 107.505044) (end 86.66 114.295) (width 0.25) (layer F.Cu) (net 60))
 (segment (start 93.899967 112.595033) (end 86.66 119.835) (width 0.25) (layer F.Cu) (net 61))
 (segment (start 93.899967 93.902788) (end 93.899967 112.595033) (width 0.25) (layer F.Cu) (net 61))
 (segment (start 87.63 74.93) (end 84.720024 77.839976) (width 0.25) (layer F.Cu) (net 61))
 (segment (start 84.720024 77.839976) (end 84.720024 84.722846) (width 0.25) (layer F.Cu) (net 61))
 (segment (start 84.720024 84.722846) (end 93.899967 93.902788) (width 0.25) (layer F.Cu) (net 61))
 (segment (start 94.349978 93.716388) (end 94.349978 117.685022) (width 0.25) (layer F.Cu) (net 62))
 (segment (start 85.170035 84.536446) (end 94.349978 93.716388) (width 0.25) (layer F.Cu) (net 62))
 (segment (start 94.349978 117.685022) (end 87.459999 124.575001) (width 0.25) (layer F.Cu) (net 62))
 (segment (start 85.170035 79.929965) (end 85.170035 84.536446) (width 0.25) (layer F.Cu) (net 62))
 (segment (start 87.459999 124.575001) (end 86.66 125.375) (width 0.25) (layer F.Cu) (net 62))
 (segment (start 87.63 77.47) (end 85.170035 79.929965) (width 0.25) (layer F.Cu) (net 62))
 (segment (start 86.66 130.915) (end 94.799989 122.775011) (width 0.25) (layer F.Cu) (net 63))
 (segment (start 85.620046 84.350046) (end 85.620046 82.019954) (width 0.25) (layer F.Cu) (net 63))
 (segment (start 94.799989 122.775011) (end 94.799989 93.529989) (width 0.25) (layer F.Cu) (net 63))
 (segment (start 94.799989 93.529989) (end 85.620046 84.350046) (width 0.25) (layer F.Cu) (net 63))
 (segment (start 85.620046 82.019954) (end 87.63 80.01) (width 0.25) (layer F.Cu) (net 63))
 (segment (start 95.25 92.71) (end 87.63 85.09) (width 0.25) (layer F.Cu) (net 67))
 (segment (start 87.63 85.09) (end 87.63 82.55) (width 0.25) (layer F.Cu) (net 67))
 (segment (start 95.25 138.945) (end 95.25 92.71) (width 0.25) (layer F.Cu) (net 67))
 (segment (start 86.66 147.535) (end 95.25 138.945) (width 0.25) (layer F.Cu) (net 67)))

